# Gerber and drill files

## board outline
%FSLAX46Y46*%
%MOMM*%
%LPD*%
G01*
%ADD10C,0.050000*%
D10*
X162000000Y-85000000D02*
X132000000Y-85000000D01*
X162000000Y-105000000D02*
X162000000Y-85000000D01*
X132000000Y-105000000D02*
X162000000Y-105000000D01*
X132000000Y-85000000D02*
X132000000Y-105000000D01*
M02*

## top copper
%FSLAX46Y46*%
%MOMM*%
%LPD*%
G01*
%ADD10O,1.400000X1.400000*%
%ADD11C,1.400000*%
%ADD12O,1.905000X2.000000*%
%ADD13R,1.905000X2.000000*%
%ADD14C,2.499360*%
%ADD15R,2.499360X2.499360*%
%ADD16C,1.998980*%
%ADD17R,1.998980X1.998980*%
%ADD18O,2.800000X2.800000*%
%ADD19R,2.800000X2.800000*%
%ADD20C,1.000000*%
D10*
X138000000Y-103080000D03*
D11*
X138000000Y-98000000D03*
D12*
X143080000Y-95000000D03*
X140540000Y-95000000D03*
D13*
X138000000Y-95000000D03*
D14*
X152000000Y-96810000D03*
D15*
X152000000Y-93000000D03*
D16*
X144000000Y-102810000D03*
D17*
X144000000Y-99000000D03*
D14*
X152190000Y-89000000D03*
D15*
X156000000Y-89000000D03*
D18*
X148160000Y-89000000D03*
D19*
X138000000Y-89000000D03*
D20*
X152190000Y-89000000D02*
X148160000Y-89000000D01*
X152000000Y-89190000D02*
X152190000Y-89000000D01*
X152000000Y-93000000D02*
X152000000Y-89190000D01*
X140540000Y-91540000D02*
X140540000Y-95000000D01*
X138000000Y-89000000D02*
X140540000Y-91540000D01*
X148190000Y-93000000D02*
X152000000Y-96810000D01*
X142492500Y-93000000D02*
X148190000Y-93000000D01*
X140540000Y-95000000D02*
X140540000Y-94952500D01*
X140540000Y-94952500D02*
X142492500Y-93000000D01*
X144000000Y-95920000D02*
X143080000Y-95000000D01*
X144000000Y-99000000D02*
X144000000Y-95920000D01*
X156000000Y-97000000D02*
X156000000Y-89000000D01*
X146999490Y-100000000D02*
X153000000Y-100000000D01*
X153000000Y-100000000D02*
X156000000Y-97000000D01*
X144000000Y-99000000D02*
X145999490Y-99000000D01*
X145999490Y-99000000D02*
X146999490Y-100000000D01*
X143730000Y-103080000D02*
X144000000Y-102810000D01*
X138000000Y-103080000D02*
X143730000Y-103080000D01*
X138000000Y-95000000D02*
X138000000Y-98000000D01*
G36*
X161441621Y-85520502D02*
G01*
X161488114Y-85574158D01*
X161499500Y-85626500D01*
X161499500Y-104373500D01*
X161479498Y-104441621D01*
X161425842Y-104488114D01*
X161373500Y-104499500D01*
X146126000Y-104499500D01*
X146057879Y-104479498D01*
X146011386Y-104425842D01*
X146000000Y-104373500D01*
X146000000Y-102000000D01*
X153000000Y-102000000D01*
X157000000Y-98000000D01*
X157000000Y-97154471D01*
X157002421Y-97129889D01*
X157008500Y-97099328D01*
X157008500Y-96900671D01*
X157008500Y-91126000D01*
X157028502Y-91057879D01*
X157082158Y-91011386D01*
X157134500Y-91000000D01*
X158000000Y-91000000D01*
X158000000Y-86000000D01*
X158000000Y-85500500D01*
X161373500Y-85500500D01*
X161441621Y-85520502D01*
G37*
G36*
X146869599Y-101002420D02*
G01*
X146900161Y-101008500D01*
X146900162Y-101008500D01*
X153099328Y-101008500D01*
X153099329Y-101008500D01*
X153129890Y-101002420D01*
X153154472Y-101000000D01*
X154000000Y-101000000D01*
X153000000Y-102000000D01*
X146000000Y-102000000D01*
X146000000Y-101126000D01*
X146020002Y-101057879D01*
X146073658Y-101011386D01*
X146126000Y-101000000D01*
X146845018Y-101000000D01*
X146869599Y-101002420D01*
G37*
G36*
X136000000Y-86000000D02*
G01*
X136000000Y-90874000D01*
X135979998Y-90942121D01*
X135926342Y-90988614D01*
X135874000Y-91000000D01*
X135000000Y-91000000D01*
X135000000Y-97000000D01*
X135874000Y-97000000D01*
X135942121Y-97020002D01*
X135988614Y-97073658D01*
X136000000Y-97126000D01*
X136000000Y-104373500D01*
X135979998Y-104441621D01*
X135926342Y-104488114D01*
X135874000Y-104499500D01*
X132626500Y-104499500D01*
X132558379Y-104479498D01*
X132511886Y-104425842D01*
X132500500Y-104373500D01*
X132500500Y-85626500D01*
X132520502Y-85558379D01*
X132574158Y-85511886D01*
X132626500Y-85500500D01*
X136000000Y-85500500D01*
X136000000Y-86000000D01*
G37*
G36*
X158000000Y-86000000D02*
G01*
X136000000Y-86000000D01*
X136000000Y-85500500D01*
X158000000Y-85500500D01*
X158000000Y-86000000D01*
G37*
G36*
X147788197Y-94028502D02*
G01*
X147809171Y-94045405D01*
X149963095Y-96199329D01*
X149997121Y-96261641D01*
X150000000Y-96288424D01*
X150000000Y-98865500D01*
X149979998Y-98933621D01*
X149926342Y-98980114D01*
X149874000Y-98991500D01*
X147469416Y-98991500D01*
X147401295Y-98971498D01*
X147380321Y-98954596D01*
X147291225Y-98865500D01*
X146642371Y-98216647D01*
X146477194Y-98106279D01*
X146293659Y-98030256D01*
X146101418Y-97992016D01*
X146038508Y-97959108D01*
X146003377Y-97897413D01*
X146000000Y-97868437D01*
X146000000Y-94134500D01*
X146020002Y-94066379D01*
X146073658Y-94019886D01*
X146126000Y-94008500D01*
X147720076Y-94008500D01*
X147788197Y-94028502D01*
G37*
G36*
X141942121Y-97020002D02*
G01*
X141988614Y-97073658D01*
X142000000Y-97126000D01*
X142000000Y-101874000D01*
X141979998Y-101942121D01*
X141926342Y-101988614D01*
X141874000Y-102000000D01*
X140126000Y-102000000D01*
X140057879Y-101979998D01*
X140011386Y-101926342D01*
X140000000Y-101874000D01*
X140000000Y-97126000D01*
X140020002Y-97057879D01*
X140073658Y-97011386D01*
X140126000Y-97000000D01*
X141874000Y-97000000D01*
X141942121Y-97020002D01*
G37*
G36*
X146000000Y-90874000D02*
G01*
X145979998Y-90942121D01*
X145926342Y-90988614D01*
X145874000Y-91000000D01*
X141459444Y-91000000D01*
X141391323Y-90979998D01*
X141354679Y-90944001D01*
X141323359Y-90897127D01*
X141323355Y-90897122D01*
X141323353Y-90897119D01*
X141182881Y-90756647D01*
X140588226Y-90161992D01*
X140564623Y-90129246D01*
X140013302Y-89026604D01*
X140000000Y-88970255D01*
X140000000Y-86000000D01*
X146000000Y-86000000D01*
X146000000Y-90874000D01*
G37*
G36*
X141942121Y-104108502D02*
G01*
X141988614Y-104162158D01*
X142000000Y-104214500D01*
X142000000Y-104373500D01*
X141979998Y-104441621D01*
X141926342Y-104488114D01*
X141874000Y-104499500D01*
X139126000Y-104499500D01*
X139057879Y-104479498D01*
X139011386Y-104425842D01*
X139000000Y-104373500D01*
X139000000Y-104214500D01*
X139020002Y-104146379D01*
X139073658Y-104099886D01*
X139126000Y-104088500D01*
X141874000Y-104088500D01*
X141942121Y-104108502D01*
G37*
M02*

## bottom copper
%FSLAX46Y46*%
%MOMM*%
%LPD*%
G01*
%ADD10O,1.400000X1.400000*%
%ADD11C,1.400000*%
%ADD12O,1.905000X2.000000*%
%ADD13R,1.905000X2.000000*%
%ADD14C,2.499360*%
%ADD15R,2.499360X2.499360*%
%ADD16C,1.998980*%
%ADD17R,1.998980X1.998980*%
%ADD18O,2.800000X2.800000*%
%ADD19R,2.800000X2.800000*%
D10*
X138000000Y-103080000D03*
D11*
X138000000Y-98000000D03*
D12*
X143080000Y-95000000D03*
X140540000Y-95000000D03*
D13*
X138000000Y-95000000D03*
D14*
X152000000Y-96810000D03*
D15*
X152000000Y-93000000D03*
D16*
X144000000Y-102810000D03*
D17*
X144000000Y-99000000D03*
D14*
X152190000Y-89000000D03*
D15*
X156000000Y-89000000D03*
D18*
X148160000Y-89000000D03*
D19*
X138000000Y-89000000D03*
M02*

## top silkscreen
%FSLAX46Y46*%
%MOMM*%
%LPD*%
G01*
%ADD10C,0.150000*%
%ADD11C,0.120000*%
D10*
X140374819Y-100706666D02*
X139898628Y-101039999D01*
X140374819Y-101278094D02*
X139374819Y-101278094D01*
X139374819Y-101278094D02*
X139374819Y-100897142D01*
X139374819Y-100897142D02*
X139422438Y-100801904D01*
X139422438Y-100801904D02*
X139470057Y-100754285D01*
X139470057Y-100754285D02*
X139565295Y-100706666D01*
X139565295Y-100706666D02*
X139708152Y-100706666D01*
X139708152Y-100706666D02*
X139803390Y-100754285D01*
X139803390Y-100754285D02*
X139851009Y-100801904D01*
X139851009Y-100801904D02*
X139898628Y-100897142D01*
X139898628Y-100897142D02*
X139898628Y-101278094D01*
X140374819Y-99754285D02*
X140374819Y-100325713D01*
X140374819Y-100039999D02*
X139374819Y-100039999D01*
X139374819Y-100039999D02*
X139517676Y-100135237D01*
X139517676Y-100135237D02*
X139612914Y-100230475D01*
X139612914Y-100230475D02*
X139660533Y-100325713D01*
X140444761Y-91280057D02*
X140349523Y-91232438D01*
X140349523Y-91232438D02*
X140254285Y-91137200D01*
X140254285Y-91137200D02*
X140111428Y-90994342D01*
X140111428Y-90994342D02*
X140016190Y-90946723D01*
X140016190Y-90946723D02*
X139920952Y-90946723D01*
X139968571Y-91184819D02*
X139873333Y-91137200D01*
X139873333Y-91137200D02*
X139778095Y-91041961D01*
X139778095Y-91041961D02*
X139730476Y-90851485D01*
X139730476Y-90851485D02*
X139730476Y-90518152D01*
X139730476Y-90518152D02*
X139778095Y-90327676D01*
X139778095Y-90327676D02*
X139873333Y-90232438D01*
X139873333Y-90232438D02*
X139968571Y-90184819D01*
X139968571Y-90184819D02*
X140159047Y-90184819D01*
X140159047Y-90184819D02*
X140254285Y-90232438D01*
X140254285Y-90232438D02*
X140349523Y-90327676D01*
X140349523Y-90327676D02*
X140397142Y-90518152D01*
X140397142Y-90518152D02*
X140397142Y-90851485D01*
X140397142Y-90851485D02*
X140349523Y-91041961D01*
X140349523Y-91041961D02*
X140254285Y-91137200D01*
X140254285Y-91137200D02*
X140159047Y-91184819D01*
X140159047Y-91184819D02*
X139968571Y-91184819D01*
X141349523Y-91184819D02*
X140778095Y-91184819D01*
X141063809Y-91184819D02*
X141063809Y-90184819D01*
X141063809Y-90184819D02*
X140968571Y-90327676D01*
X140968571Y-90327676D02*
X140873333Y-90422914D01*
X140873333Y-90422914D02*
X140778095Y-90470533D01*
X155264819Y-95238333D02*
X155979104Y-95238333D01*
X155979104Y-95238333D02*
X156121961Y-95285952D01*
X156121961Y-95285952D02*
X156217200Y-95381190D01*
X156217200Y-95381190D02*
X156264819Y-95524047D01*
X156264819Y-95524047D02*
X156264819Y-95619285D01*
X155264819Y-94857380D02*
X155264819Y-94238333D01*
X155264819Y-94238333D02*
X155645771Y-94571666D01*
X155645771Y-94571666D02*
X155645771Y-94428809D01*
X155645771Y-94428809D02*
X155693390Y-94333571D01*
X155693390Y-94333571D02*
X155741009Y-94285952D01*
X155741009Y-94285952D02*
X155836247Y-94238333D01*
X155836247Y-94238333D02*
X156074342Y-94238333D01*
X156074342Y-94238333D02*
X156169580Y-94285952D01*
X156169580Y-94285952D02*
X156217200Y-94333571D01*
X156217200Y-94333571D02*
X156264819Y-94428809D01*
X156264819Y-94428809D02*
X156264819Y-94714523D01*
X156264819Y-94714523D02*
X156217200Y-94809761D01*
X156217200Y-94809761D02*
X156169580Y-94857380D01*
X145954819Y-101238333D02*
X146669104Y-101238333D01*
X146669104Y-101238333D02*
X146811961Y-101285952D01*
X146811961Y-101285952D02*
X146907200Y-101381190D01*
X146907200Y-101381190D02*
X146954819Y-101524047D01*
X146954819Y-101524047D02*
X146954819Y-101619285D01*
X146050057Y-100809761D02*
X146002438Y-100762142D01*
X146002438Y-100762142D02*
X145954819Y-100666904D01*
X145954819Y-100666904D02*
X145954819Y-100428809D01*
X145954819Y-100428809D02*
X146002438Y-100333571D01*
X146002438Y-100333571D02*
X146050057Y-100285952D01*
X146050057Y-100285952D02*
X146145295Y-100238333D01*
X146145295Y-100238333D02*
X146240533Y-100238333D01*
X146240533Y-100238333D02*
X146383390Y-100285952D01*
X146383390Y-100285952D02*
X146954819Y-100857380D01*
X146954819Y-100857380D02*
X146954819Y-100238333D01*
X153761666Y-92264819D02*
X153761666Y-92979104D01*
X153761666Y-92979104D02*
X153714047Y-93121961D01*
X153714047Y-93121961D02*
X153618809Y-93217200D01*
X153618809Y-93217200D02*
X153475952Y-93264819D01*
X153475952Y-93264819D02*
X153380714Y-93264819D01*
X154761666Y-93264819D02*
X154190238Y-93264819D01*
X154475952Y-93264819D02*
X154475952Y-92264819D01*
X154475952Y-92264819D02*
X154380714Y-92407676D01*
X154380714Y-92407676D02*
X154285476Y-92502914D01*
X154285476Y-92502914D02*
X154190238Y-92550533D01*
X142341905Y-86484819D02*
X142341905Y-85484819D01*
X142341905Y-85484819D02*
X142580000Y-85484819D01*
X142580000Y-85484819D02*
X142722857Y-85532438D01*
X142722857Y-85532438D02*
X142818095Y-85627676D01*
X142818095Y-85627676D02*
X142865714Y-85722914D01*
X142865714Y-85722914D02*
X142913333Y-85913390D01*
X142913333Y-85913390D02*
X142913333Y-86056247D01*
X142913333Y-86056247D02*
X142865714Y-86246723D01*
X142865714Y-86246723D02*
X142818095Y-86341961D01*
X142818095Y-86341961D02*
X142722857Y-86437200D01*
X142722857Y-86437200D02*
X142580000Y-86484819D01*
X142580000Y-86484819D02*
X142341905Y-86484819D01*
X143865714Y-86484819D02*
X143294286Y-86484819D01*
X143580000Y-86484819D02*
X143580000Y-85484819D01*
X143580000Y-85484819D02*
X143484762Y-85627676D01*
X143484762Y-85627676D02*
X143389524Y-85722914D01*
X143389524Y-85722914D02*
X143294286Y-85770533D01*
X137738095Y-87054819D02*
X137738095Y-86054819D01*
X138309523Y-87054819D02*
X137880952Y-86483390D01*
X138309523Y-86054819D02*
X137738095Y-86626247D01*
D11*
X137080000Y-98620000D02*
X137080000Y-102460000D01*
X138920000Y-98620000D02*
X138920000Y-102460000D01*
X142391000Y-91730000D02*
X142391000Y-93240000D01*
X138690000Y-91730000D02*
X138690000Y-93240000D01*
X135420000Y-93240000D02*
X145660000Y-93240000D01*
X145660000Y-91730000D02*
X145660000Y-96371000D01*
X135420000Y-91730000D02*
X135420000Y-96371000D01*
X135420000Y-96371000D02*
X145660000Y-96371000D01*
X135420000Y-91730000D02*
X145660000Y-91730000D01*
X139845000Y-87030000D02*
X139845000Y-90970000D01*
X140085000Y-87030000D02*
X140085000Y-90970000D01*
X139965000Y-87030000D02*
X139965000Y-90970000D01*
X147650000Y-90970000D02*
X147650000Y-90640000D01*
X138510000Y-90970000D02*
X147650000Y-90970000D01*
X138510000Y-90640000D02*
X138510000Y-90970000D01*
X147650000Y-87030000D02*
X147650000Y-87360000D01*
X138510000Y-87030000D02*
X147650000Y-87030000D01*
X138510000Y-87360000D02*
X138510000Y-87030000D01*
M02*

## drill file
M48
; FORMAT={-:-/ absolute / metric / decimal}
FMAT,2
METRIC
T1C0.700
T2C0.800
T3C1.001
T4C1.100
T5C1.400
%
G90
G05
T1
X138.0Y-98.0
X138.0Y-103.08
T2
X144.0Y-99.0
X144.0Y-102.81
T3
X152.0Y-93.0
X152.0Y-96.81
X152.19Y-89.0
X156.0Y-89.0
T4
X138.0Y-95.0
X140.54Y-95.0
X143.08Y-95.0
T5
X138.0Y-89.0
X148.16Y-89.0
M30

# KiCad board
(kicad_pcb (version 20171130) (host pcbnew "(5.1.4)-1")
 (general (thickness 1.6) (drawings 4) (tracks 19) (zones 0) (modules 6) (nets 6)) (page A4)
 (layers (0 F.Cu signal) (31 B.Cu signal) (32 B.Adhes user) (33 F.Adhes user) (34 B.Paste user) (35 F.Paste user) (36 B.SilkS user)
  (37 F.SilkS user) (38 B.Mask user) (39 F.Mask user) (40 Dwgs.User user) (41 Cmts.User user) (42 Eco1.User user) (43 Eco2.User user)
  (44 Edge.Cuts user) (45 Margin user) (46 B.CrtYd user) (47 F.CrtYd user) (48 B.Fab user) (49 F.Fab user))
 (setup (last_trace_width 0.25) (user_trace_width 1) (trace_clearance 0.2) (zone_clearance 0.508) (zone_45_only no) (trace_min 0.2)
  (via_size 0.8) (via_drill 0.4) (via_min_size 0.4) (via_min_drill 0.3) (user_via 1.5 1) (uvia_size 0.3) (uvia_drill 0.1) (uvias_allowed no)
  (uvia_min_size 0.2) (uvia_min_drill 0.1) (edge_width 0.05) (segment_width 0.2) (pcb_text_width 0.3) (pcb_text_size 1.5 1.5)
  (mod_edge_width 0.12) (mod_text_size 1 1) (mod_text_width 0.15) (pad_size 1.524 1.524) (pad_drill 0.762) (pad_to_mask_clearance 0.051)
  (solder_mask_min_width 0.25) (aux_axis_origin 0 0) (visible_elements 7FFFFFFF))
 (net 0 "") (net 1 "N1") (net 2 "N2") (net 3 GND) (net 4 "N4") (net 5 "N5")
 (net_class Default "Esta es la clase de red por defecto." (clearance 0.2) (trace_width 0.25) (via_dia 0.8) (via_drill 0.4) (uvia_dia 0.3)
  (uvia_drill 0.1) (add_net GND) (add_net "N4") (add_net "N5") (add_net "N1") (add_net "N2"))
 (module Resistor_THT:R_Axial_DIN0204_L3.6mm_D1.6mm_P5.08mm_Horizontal (layer F.Cu) (at 138 98 270)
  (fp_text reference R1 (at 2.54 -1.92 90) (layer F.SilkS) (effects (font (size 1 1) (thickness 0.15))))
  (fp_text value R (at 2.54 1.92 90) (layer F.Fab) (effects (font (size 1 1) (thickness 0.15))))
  (fp_line (start 0.62 0.92) (end 4.46 0.92) (layer F.SilkS) (width 0.12))
  (fp_line (start 0.62 -0.92) (end 4.46 -0.92) (layer F.SilkS) (width 0.12))
  (pad 2 thru_hole oval (at 5.08 0 270) (size 1.4 1.4) (drill 0.7) (layers *.Cu *.Mask) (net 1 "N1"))
  (pad 1 thru_hole circle (at 0 0 270) (size 1.4 1.4) (drill 0.7) (layers *.Cu *.Mask) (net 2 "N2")))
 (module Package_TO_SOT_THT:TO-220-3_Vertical (layer F.Cu) (at 138 95)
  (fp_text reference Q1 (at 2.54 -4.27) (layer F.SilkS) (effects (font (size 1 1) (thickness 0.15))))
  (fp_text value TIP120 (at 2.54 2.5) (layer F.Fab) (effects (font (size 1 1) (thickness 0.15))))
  (fp_line (start 4.391 -3.27) (end 4.391 -1.76) (layer F.SilkS) (width 0.12))
  (fp_line (start 0.69 -3.27) (end 0.69 -1.76) (layer F.SilkS) (width 0.12))
  (fp_line (start -2.58 -1.76) (end 7.66 -1.76) (layer F.SilkS) (width 0.12))
  (fp_line (start 7.66 -3.27) (end 7.66 1.371) (layer F.SilkS) (width 0.12))
  (fp_line (start -2.58 -3.27) (end -2.58 1.371) (layer F.SilkS) (width 0.12))
  (fp_line (start -2.58 1.371) (end 7.66 1.371) (layer F.SilkS) (width 0.12))
  (fp_line (start -2.58 -3.27) (end 7.66 -3.27) (layer F.SilkS) (width 0.12))
  (pad 3 thru_hole oval (at 5.08 0) (size 1.905 2) (drill 1.1) (layers *.Cu *.Mask) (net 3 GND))
  (pad 2 thru_hole oval (at 2.54 0) (size 1.905 2) (drill 1.1) (layers *.Cu *.Mask) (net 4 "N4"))
  (pad 1 thru_hole rect (at 0 0) (size 1.905 2) (drill 1.1) (layers *.Cu *.Mask) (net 2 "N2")))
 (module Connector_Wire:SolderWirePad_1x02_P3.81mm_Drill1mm (layer F.Cu) (at 152 93 270)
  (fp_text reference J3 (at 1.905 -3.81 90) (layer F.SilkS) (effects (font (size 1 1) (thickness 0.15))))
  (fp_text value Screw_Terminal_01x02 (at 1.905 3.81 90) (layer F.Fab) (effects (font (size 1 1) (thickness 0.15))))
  (pad 2 thru_hole circle (at 3.81 0 270) (size 2.49936 2.49936) (drill 1.00076) (layers *.Cu *.Mask) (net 4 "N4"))
  (pad 1 thru_hole rect (at 0 0 270) (size 2.49936 2.49936) (drill 1.00076) (layers *.Cu *.Mask) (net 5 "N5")))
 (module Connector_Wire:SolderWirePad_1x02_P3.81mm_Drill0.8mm (layer F.Cu) (at 144 99 270)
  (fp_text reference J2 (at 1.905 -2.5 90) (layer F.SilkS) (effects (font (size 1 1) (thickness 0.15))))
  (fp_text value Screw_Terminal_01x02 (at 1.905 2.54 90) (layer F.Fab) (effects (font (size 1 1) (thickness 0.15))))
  (pad 2 thru_hole circle (at 3.81 0 270) (size 1.99898 1.99898) (drill 0.8001) (layers *.Cu *.Mask) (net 1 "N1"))
  (pad 1 thru_hole rect (at 0 0 270) (size 1.99898 1.99898) (drill 0.8001) (layers *.Cu *.Mask) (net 3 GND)))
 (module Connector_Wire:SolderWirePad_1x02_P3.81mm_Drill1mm (layer F.Cu) (at 156 89 180)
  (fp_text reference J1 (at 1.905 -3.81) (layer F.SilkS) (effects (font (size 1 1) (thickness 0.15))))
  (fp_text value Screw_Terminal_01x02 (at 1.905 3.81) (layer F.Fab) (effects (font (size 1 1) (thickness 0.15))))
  (pad 2 thru_hole circle (at 3.81 0 180) (size 2.49936 2.49936) (drill 1.00076) (layers *.Cu *.Mask) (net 5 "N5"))
  (pad 1 thru_hole rect (at 0 0 180) (size 2.49936 2.49936) (drill 1.00076) (layers *.Cu *.Mask) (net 3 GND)))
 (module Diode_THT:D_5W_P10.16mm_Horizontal (layer F.Cu) (at 138 89)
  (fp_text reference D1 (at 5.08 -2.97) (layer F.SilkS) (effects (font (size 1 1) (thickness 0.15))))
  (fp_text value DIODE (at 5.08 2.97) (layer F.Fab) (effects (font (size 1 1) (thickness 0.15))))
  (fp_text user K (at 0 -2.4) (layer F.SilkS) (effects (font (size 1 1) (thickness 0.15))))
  (fp_line (start 1.845 -1.97) (end 1.845 1.97) (layer F.SilkS) (width 0.12))
  (fp_line (start 2.085 -1.97) (end 2.085 1.97) (layer F.SilkS) (width 0.12))
  (fp_line (start 1.965 -1.97) (end 1.965 1.97) (layer F.SilkS) (width 0.12))
  (fp_line (start 9.65 1.97) (end 9.65 1.64) (layer F.SilkS) (width 0.12))
  (fp_line (start 0.51 1.97) (end 9.65 1.97) (layer F.SilkS) (width 0.12))
  (fp_line (start 0.51 1.64) (end 0.51 1.97) (layer F.SilkS) (width 0.12))
  (fp_line (start 9.65 -1.97) (end 9.65 -1.64) (layer F.SilkS) (width 0.12))
  (fp_line (start 0.51 -1.97) (end 9.65 -1.97) (layer F.SilkS) (width 0.12))
  (fp_line (start 0.51 -1.64) (end 0.51 -1.97) (layer F.SilkS) (width 0.12))
  (pad 2 thru_hole oval (at 10.16 0) (size 2.8 2.8) (drill 1.4) (layers *.Cu *.Mask) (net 5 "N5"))
  (pad 1 thru_hole rect (at 0 0) (size 2.8 2.8) (drill 1.4) (layers *.Cu *.Mask) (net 4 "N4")))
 (gr_line (start 162 85) (end 132 85) (layer Edge.Cuts) (width 0.05))
 (gr_line (start 162 105) (end 162 85) (layer Edge.Cuts) (width 0.05))
 (gr_line (start 132 105) (end 162 105) (layer Edge.Cuts) (width 0.05))
 (gr_line (start 132 85) (end 132 105) (layer Edge.Cuts) (width 0.05))
 (segment (start 152.19 89) (end 148.16 89) (width 1) (layer F.Cu) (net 5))
 (segment (start 152 89.19) (end 152.19 89) (width 1) (layer F.Cu) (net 5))
 (segment (start 152 93) (end 152 89.19) (width 1) (layer F.Cu) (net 5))
 (segment (start 140.54 91.54) (end 140.54 95) (width 1) (layer F.Cu) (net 4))
 (segment (start 138 89) (end 140.54 91.54) (width 1) (layer F.Cu) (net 4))
 (segment (start 148.19 93) (end 152 96.81) (width 1) (layer F.Cu) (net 4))
 (segment (start 142.4925 93) (end 148.19 93) (width 1) (layer F.Cu) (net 4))
 (segment (start 140.54 95) (end 140.54 94.9525) (width 1) (layer F.Cu) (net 4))
 (segment (start 140.54 94.9525) (end 142.4925 93) (width 1) (layer F.Cu) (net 4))
 (segment (start 144 95.92) (end 143.08 95) (width 1) (layer F.Cu) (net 3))
 (segment (start 144 99) (end 144 95.92) (width 1) (layer F.Cu) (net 3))
 (segment (start 156 97) (end 156 89) (width 1) (layer F.Cu) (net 3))
 (segment (start 146.99949 100) (end 153 100) (width 1) (layer F.Cu) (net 3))
 (segment (start 153 100) (end 156 97) (width 1) (layer F.Cu) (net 3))
 (segment (start 144 99) (end 145.99949 99) (width 1) (layer F.Cu) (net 3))
 (segment (start 145.99949 99) (end 146.99949 100) (width 1) (layer F.Cu) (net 3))
 (segment (start 143.73 103.08) (end 144 102.81) (width 1) (layer F.Cu) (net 1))
 (segment (start 138 103.08) (end 143.73 103.08) (width 1) (layer F.Cu) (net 1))
 (segment (start 138 95) (end 138 98) (width 1) (layer F.Cu) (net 2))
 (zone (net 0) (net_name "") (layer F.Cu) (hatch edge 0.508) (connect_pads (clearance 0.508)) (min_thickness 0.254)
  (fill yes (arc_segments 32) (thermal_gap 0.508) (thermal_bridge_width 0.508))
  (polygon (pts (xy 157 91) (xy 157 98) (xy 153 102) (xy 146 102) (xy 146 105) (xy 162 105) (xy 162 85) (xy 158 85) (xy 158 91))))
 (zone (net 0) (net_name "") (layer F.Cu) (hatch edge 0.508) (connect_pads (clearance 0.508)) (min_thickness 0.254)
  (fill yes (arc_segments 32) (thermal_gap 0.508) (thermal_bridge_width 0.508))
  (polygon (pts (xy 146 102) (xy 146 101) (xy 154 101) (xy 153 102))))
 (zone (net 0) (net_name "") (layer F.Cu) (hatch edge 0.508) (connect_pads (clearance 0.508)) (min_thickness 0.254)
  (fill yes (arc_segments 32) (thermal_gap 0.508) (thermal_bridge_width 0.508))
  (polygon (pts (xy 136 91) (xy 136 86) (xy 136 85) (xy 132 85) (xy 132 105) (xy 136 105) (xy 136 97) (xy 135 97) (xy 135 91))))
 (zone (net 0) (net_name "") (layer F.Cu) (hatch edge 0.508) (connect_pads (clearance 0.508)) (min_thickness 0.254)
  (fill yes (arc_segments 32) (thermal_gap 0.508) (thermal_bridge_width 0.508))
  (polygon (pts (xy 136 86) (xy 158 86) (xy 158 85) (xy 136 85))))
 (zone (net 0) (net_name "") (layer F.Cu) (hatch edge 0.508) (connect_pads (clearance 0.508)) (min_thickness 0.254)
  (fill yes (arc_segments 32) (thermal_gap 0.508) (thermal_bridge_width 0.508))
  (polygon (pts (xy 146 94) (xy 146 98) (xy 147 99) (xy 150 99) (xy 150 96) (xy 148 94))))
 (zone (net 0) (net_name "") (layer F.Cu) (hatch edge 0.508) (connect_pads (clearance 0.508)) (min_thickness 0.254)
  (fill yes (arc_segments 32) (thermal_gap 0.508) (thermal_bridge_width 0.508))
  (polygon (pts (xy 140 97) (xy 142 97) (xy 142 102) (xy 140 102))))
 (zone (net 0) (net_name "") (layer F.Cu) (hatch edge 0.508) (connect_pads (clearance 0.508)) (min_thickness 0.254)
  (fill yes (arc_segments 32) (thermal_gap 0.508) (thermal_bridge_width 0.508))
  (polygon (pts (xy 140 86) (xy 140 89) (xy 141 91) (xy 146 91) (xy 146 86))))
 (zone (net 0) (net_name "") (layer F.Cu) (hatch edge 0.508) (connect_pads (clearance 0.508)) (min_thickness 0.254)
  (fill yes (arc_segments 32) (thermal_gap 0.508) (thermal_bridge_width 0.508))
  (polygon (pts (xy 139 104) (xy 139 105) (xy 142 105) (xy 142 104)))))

